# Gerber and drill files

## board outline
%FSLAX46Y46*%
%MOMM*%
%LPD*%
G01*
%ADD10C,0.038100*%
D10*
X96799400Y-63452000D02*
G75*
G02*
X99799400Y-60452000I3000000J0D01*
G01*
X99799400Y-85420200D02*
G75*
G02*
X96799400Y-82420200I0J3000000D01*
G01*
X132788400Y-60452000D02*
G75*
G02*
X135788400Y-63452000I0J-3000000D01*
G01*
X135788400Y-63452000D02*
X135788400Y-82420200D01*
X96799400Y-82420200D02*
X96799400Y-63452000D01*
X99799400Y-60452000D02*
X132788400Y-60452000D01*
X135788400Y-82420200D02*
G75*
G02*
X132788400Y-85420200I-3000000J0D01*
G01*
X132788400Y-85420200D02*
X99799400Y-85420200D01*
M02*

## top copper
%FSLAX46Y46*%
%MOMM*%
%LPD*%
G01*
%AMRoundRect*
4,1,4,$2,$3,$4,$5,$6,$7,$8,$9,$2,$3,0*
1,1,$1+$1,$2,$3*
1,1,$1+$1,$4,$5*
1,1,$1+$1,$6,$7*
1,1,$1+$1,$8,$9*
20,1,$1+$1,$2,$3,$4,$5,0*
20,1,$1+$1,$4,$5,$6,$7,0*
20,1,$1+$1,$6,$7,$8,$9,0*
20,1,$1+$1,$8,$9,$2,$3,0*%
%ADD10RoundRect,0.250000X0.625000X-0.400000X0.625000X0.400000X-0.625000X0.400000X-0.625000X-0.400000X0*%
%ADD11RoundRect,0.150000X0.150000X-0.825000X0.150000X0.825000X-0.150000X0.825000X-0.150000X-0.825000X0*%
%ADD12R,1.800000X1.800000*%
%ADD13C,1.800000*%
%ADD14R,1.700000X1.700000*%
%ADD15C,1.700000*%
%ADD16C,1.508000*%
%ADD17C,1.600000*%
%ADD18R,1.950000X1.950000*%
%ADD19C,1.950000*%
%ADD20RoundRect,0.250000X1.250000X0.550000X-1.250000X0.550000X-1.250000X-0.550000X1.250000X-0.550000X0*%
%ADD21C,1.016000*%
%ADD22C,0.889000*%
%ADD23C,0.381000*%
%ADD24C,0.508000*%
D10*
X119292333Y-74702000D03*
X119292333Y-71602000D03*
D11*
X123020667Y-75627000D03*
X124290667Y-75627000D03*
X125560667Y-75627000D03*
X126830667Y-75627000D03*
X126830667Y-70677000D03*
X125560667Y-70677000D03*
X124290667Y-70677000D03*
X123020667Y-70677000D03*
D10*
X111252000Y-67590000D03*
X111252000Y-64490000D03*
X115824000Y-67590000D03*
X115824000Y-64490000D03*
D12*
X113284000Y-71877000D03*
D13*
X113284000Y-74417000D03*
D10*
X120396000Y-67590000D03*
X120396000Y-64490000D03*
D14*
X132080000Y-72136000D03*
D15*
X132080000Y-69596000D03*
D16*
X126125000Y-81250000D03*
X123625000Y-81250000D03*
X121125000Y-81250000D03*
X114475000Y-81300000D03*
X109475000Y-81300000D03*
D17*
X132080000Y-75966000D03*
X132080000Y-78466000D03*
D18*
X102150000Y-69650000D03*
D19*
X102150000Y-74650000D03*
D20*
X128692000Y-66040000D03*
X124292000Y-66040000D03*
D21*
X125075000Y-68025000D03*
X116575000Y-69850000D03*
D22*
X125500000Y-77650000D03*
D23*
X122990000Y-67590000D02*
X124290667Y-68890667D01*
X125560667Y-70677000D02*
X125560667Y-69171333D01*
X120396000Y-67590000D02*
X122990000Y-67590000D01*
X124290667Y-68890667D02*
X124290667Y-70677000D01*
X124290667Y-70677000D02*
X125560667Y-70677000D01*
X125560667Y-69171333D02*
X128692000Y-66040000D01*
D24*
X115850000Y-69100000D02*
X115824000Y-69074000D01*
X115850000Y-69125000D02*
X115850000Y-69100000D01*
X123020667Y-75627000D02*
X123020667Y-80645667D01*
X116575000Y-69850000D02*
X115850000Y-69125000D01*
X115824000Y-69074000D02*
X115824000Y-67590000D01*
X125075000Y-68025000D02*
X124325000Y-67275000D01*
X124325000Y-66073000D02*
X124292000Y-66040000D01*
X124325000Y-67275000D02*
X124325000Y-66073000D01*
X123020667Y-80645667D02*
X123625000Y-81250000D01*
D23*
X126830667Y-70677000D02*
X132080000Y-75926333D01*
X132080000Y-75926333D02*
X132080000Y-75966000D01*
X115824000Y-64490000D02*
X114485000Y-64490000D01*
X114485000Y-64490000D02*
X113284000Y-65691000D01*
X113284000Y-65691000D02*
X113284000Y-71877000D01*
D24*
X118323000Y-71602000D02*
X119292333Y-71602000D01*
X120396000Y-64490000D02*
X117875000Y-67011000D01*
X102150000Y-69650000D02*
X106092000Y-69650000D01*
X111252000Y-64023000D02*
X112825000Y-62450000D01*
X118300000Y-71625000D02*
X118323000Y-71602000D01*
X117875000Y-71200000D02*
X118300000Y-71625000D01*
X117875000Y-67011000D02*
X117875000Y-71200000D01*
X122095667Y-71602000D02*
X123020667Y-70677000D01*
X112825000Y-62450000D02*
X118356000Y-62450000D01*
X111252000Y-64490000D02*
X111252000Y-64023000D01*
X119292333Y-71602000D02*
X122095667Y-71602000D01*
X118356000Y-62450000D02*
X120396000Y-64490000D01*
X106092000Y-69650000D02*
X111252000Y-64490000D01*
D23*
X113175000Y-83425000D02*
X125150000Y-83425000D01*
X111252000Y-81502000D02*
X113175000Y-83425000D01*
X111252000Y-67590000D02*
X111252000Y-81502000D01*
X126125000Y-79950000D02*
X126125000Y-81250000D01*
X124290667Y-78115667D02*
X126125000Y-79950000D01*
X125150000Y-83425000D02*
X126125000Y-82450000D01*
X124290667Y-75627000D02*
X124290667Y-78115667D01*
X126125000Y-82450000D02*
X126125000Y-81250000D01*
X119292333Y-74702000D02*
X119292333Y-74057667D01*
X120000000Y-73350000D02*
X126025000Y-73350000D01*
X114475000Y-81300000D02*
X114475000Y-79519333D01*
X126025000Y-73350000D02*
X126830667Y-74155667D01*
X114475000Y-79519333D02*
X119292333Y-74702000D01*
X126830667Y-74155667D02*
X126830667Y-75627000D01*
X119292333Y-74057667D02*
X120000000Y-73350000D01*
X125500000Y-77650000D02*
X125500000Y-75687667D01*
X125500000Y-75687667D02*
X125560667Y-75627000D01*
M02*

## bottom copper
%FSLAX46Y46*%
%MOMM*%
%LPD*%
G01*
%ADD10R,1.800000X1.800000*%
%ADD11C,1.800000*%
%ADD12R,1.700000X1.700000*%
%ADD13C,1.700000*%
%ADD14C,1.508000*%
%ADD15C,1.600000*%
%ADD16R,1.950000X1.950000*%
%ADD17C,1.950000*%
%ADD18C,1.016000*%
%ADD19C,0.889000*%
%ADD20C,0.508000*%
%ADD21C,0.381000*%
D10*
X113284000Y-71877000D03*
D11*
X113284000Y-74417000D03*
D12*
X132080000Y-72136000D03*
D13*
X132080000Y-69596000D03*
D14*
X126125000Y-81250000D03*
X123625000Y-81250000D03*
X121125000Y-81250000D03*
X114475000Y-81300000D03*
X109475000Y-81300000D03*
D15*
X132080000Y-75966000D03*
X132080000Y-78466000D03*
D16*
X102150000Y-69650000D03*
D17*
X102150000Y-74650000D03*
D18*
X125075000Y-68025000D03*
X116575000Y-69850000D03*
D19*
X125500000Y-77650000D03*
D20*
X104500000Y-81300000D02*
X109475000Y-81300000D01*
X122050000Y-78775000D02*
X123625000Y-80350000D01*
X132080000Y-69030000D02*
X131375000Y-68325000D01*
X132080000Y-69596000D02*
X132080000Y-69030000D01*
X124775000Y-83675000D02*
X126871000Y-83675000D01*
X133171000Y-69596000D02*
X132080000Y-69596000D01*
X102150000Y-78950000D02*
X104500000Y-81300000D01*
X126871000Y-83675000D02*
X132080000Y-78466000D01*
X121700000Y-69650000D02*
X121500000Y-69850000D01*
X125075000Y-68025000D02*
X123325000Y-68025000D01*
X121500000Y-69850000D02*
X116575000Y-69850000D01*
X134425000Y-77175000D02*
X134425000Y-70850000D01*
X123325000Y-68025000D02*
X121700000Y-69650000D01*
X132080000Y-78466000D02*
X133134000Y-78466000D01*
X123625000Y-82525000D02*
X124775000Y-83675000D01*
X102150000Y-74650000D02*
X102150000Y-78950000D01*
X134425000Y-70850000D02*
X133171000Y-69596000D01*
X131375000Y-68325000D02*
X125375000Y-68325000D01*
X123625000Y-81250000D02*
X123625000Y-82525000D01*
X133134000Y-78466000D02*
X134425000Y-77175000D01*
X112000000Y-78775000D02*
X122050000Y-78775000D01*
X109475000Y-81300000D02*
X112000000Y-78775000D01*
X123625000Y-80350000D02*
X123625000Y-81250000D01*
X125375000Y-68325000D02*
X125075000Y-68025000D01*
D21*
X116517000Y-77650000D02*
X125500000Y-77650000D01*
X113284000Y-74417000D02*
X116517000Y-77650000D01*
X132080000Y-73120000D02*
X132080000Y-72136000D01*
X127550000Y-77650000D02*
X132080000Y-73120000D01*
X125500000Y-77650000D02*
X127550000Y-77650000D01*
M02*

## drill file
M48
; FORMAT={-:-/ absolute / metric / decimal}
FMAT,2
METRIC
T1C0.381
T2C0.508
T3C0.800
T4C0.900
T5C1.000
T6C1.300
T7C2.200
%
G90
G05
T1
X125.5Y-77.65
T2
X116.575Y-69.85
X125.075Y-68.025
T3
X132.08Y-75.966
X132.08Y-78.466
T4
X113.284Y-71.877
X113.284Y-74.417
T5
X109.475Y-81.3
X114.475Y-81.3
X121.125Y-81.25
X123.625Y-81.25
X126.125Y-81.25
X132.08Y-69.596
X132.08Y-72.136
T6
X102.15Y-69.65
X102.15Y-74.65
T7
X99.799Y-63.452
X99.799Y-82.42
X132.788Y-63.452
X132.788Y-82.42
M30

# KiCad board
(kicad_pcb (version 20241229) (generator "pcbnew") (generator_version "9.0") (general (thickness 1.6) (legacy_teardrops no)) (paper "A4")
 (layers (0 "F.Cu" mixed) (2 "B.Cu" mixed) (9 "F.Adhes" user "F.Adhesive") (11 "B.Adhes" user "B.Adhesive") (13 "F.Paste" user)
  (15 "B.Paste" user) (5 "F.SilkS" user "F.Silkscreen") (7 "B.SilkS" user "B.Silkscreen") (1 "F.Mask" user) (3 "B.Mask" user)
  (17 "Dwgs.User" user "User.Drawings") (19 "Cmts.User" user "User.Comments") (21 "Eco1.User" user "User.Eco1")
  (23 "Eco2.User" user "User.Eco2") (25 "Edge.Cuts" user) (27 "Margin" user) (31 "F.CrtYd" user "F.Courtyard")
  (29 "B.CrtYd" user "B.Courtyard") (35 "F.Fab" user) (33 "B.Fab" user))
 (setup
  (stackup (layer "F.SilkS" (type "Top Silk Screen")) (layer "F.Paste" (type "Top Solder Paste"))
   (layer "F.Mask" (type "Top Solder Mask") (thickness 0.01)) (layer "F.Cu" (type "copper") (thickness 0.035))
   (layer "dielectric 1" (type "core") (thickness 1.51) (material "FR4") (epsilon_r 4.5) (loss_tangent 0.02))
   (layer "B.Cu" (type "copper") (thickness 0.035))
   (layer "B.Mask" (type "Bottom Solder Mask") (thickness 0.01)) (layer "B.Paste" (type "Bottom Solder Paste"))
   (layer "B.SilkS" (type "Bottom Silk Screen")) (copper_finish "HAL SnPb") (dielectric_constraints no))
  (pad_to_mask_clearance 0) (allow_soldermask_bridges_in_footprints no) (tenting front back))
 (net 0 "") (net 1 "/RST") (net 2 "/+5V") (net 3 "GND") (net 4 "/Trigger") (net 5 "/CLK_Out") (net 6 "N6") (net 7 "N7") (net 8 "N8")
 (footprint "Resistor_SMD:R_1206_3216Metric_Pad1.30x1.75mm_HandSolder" (layer "F.Cu") (at 119.292333 73.152 90)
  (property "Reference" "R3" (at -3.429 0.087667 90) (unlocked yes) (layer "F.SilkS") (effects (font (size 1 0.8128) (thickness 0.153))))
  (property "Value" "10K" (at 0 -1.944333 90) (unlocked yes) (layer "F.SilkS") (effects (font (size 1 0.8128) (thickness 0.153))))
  (pad "1" smd roundrect (at -1.55 0 90) (size 1.3 1.75) (layers "F.Cu" "F.Mask" "F.Paste") (roundrect_rratio 0.192308) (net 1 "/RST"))
  (pad "2" smd roundrect (at 1.55 0 90) (size 1.3 1.75) (layers "F.Cu" "F.Mask" "F.Paste") (roundrect_rratio 0.192308) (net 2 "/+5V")))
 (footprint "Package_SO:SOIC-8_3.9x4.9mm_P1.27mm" (layer "F.Cu") (at 124.925667 73.152 90)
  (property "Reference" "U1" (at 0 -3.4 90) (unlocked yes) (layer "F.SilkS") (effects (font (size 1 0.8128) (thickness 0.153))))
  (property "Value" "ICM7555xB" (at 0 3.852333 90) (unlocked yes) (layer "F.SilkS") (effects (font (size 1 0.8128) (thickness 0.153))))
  (pad "1" smd roundrect (at -2.475 -1.905 90) (size 1.95 0.6) (layers "F.Cu" "F.Mask" "F.Paste") (roundrect_rratio 0.25) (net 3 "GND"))
  (pad "2" smd roundrect (at -2.475 -0.635 90) (size 1.95 0.6) (layers "F.Cu" "F.Mask" "F.Paste") (roundrect_rratio 0.25) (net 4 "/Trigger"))
  (pad "3" smd roundrect (at -2.475 0.635 90) (size 1.95 0.6) (layers "F.Cu" "F.Mask" "F.Paste") (roundrect_rratio 0.25) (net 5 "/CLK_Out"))
  (pad "4" smd roundrect (at -2.475 1.905 90) (size 1.95 0.6) (layers "F.Cu" "F.Mask" "F.Paste") (roundrect_rratio 0.25) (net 1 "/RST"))
  (pad "5" smd roundrect (at 2.475 1.905 90) (size 1.95 0.6) (layers "F.Cu" "F.Mask" "F.Paste") (roundrect_rratio 0.25) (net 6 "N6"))
  (pad "6" smd roundrect (at 2.475 0.635 90) (size 1.95 0.6) (layers "F.Cu" "F.Mask" "F.Paste") (roundrect_rratio 0.25) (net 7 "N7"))
  (pad "7" smd roundrect (at 2.475 -0.635 90) (size 1.95 0.6) (layers "F.Cu" "F.Mask" "F.Paste") (roundrect_rratio 0.25) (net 7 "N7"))
  (pad "8" smd roundrect (at 2.475 -1.905 90) (size 1.95 0.6) (layers "F.Cu" "F.Mask" "F.Paste") (roundrect_rratio 0.25) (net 2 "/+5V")))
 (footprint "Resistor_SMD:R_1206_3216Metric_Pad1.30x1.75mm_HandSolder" (layer "F.Cu") (at 111.252 66.04 90)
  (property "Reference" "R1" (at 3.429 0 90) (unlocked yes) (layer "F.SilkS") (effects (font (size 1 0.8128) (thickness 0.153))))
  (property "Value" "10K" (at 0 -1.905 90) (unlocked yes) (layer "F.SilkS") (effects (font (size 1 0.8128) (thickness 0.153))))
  (pad "1" smd roundrect (at -1.55 0 90) (size 1.3 1.75) (layers "F.Cu" "F.Mask" "F.Paste") (roundrect_rratio 0.192308) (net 4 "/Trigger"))
  (pad "2" smd roundrect (at 1.55 0 90) (size 1.3 1.75) (layers "F.Cu" "F.Mask" "F.Paste") (roundrect_rratio 0.192308) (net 2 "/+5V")))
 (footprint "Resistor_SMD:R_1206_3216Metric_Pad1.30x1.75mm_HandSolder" (layer "F.Cu") (at 115.824 66.04 90)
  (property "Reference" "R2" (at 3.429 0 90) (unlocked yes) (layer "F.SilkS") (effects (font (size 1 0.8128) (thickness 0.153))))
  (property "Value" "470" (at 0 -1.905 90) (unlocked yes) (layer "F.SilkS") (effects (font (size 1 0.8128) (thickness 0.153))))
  (pad "1" smd roundrect (at -1.55 0 90) (size 1.3 1.75) (layers "F.Cu" "F.Mask" "F.Paste") (roundrect_rratio 0.192308) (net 3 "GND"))
  (pad "2" smd roundrect (at 1.55 0 90) (size 1.3 1.75) (layers "F.Cu" "F.Mask" "F.Paste") (roundrect_rratio 0.192308) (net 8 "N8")))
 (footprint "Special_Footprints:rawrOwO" (layer "F.Cu") (at 105.7 63.275)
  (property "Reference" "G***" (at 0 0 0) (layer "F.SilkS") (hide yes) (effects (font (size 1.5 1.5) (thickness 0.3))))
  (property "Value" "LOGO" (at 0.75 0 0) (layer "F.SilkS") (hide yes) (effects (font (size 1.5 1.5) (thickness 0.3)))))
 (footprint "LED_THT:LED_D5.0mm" (layer "F.Cu") (at 113.284 71.877 -90)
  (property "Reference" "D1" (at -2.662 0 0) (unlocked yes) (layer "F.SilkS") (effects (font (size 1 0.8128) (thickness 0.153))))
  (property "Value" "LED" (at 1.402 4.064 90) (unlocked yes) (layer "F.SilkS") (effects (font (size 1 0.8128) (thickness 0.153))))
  (pad "1" thru_hole rect (at 0 0 270) (size 1.8 1.8) (drill 0.9) (layers "*.Cu" "*.Mask") (remove_unused_layers no) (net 8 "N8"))
  (pad "2" thru_hole circle (at 2.54 0 270) (size 1.8 1.8) (drill 0.9) (layers "*.Cu" "*.Mask") (remove_unused_layers no) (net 5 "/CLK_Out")))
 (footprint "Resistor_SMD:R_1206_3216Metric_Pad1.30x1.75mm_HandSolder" (layer "F.Cu") (at 120.396 66.04 90)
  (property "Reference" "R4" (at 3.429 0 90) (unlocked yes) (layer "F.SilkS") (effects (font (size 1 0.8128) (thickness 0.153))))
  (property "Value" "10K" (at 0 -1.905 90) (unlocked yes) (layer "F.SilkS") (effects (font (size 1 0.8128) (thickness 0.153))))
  (pad "1" smd roundrect (at -1.55 0 90) (size 1.3 1.75) (layers "F.Cu" "F.Mask" "F.Paste") (roundrect_rratio 0.192308) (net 7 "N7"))
  (pad "2" smd roundrect (at 1.55 0 90) (size 1.3 1.75) (layers "F.Cu" "F.Mask" "F.Paste") (roundrect_rratio 0.192308) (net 2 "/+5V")))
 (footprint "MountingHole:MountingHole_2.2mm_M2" (layer "F.Cu") (at 99.7994 63.452)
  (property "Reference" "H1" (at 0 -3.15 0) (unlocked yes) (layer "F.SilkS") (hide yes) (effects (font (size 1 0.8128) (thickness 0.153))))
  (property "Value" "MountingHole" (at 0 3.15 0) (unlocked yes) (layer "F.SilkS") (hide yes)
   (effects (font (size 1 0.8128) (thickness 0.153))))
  (pad "" np_thru_hole circle (at 0 0) (size 2.2 2.2) (drill 2.2) (layers "*.Cu" "*.Mask")))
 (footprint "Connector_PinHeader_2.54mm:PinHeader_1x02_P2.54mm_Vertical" (layer "F.Cu") (at 132.08 72.136 180)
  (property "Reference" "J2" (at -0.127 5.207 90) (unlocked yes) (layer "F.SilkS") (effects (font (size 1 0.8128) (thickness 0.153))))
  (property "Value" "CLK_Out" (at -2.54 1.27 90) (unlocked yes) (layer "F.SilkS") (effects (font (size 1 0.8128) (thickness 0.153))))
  (pad "1" thru_hole rect (at 0 0 180) (size 1.7 1.7) (drill 1) (layers "*.Cu" "*.Mask") (remove_unused_layers no) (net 5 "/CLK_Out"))
  (pad "2" thru_hole circle (at 0 2.54 180) (size 1.7 1.7) (drill 1) (layers "*.Cu" "*.Mask") (remove_unused_layers no) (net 3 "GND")))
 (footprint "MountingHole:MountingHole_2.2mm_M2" (layer "F.Cu") (at 132.7884 82.4202)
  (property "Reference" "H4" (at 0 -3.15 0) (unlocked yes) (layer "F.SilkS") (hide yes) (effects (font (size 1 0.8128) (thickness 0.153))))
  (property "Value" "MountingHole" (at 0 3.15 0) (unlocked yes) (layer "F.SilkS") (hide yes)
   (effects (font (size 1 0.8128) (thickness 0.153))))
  (pad "" np_thru_hole circle (at 0 0) (size 2.2 2.2) (drill 2.2) (layers "*.Cu" "*.Mask")))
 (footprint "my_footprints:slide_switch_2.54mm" (layer "F.Cu") (at 123.625 81.25 180)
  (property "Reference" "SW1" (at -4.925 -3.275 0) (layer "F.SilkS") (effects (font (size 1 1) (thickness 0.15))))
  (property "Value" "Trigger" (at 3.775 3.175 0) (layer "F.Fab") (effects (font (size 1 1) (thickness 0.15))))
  (pad "1" thru_hole circle (at -2.5 0 180) (size 1.508 1.508) (drill 1) (layers "*.Cu" "*.Mask") (remove_unused_layers no)
   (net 4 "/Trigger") (solder_mask_margin 0.102))
  (pad "2" thru_hole circle (at 0 0 180) (size 1.508 1.508) (drill 1) (layers "*.Cu" "*.Mask") (remove_unused_layers no) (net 3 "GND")
   (solder_mask_margin 0.102))
  (pad "3" thru_hole circle (at 2.5 0 180) (size 1.508 1.508) (drill 1) (layers "*.Cu" "*.Mask") (remove_unused_layers no)
   (solder_mask_margin 0.102)))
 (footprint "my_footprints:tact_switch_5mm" (layer "F.Cu") (at 111.975 81.3 180)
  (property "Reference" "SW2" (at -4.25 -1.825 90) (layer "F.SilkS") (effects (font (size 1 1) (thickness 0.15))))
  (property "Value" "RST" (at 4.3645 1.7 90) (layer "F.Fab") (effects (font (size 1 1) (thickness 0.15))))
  (pad "1" thru_hole circle (at -2.5 0 180) (size 1.508 1.508) (drill 1) (layers "*.Cu" "*.Mask") (remove_unused_layers no) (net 1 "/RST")
   (solder_mask_margin 0.102))
  (pad "2" thru_hole circle (at 2.5 0 180) (size 1.508 1.508) (drill 1) (layers "*.Cu" "*.Mask") (remove_unused_layers no) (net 3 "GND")
   (solder_mask_margin 0.102)))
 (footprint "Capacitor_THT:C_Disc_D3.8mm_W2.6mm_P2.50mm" (layer "F.Cu") (at 132.08 75.966 -90)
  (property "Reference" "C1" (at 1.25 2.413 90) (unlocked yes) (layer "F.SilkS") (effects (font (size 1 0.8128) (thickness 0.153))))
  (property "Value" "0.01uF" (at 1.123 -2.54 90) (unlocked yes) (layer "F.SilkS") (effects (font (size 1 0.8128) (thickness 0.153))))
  (pad "1" thru_hole circle (at 0 0 270) (size 1.6 1.6) (drill 0.8) (layers "*.Cu" "*.Mask") (remove_unused_layers no) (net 6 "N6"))
  (pad "2" thru_hole circle (at 2.5 0 270) (size 1.6 1.6) (drill 0.8) (layers "*.Cu" "*.Mask") (remove_unused_layers no) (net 3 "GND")))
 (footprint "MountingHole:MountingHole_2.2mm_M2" (layer "F.Cu") (at 132.7884 63.452)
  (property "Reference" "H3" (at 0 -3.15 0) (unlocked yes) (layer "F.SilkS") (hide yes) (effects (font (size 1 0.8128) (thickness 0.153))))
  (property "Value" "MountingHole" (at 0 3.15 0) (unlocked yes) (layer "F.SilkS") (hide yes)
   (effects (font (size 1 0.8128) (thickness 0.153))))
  (pad "" np_thru_hole circle (at 0 0) (size 2.2 2.2) (drill 2.2) (layers "*.Cu" "*.Mask")))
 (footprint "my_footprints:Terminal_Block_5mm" (layer "F.Cu") (at 102.15 72.15 -90)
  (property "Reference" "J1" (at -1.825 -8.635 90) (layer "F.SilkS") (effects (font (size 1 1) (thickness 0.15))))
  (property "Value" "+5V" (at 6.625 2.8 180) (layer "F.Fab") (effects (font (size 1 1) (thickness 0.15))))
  (pad "1" thru_hole rect (at -2.5 0 270) (size 1.95 1.95) (drill 1.3) (layers "*.Cu" "*.Mask") (remove_unused_layers no) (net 2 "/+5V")
   (solder_mask_margin 0.102))
  (pad "2" thru_hole circle (at 2.5 0 270) (size 1.95 1.95) (drill 1.3) (layers "*.Cu" "*.Mask") (remove_unused_layers no) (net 3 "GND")
   (solder_mask_margin 0.102)))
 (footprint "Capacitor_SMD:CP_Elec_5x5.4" (layer "F.Cu") (at 126.492 66.04 180)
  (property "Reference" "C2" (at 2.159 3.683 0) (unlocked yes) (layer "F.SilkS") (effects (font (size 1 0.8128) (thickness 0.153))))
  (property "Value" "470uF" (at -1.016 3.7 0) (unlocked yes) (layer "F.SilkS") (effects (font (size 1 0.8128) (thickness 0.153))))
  (pad "1" smd roundrect (at -2.2 0 180) (size 3 1.6) (layers "F.Cu" "F.Mask" "F.Paste") (roundrect_rratio 0.15625) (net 7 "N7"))
  (pad "2" smd roundrect (at 2.2 0 180) (size 3 1.6) (layers "F.Cu" "F.Mask" "F.Paste") (roundrect_rratio 0.15625) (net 3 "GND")))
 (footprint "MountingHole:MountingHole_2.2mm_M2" (layer "F.Cu") (at 99.7994 82.4202)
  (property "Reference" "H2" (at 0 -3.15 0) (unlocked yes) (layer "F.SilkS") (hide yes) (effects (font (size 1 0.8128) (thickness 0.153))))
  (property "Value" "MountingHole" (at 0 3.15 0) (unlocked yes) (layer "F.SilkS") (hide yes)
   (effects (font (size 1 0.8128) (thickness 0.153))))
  (pad "" np_thru_hole circle (at 0 0) (size 2.2 2.2) (drill 2.2) (layers "*.Cu" "*.Mask")))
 (gr_arc (start 96.7994 63.452) (mid 97.67808 61.33068) (end 99.7994 60.452) (stroke (width 0.0381) (type default)) (layer "Edge.Cuts"))
 (gr_arc (start 99.7994 85.4202) (mid 97.67808 84.54152) (end 96.7994 82.4202) (stroke (width 0.0381) (type default)) (layer "Edge.Cuts"))
 (gr_arc (start 132.7884 60.452) (mid 134.90972 61.33068) (end 135.7884 63.452) (stroke (width 0.0381) (type default)) (layer "Edge.Cuts"))
 (gr_line (start 135.7884 63.452) (end 135.7884 82.4202) (stroke (width 0.0381) (type default)) (layer "Edge.Cuts"))
 (gr_line (start 96.7994 82.4202) (end 96.7994 63.452) (stroke (width 0.0381) (type default)) (layer "Edge.Cuts"))
 (gr_line (start 99.7994 60.452) (end 132.7884 60.452) (stroke (width 0.0381) (type default)) (layer "Edge.Cuts"))
 (gr_arc (start 135.7884 82.4202) (mid 134.90972 84.54152) (end 132.7884 85.4202) (stroke (width 0.0381) (type default)) (layer "Edge.Cuts"))
 (gr_line (start 132.7884 85.4202) (end 99.7994 85.4202) (stroke (width 0.0381) (type default)) (layer "Edge.Cuts"))
 (segment (start 122.99 67.59) (end 124.290667 68.890667) (width 0.381) (layer "F.Cu") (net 7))
 (segment (start 125.560667 70.677) (end 125.560667 69.171333) (width 0.381) (layer "F.Cu") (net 7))
 (segment (start 120.396 67.59) (end 122.99 67.59) (width 0.381) (layer "F.Cu") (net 7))
 (segment (start 124.290667 68.890667) (end 124.290667 70.677) (width 0.381) (layer "F.Cu") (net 7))
 (segment (start 124.290667 70.677) (end 125.560667 70.677) (width 0.381) (layer "F.Cu") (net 7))
 (segment (start 125.560667 69.171333) (end 128.692 66.04) (width 0.381) (layer "F.Cu") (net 7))
 (segment (start 115.85 69.1) (end 115.824 69.074) (width 0.508) (layer "F.Cu") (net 3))
 (segment (start 115.85 69.125) (end 115.85 69.1) (width 0.508) (layer "F.Cu") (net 3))
 (segment (start 123.020667 75.627) (end 123.020667 80.645667) (width 0.508) (layer "F.Cu") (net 3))
 (segment (start 116.575 69.85) (end 115.85 69.125) (width 0.508) (layer "F.Cu") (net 3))
 (segment (start 115.824 69.074) (end 115.824 67.59) (width 0.508) (layer "F.Cu") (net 3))
 (segment (start 125.075 68.025) (end 124.325 67.275) (width 0.508) (layer "F.Cu") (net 3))
 (segment (start 124.325 66.073) (end 124.292 66.04) (width 0.508) (layer "F.Cu") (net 3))
 (segment (start 124.325 67.275) (end 124.325 66.073) (width 0.508) (layer "F.Cu") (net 3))
 (segment (start 123.020667 80.645667) (end 123.625 81.25) (width 0.508) (layer "F.Cu") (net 3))
 (via (at 125.075 68.025) (size 1.016) (drill 0.508) (layers "F.Cu" "B.Cu") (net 3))
 (via (at 116.575 69.85) (size 1.016) (drill 0.508) (layers "F.Cu" "B.Cu") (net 3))
 (segment (start 104.5 81.3) (end 109.475 81.3) (width 0.508) (layer "B.Cu") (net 3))
 (segment (start 122.05 78.775) (end 123.625 80.35) (width 0.508) (layer "B.Cu") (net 3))
 (segment (start 132.08 69.03) (end 131.375 68.325) (width 0.508) (layer "B.Cu") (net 3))
 (segment (start 132.08 69.596) (end 132.08 69.03) (width 0.508) (layer "B.Cu") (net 3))
 (segment (start 124.775 83.675) (end 126.871 83.675) (width 0.508) (layer "B.Cu") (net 3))
 (segment (start 133.171 69.596) (end 132.08 69.596) (width 0.508) (layer "B.Cu") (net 3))
 (segment (start 102.15 78.95) (end 104.5 81.3) (width 0.508) (layer "B.Cu") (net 3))
 (segment (start 126.871 83.675) (end 132.08 78.466) (width 0.508) (layer "B.Cu") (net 3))
 (segment (start 121.7 69.65) (end 121.5 69.85) (width 0.508) (layer "B.Cu") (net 3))
 (segment (start 125.075 68.025) (end 123.325 68.025) (width 0.508) (layer "B.Cu") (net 3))
 (segment (start 121.5 69.85) (end 116.575 69.85) (width 0.508) (layer "B.Cu") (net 3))
 (segment (start 134.425 77.175) (end 134.425 70.85) (width 0.508) (layer "B.Cu") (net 3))
 (segment (start 123.325 68.025) (end 121.7 69.65) (width 0.508) (layer "B.Cu") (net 3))
 (segment (start 132.08 78.466) (end 133.134 78.466) (width 0.508) (layer "B.Cu") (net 3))
 (segment (start 123.625 82.525) (end 124.775 83.675) (width 0.508) (layer "B.Cu") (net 3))
 (segment (start 102.15 74.65) (end 102.15 78.95) (width 0.508) (layer "B.Cu") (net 3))
 (segment (start 134.425 70.85) (end 133.171 69.596) (width 0.508) (layer "B.Cu") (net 3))
 (segment (start 131.375 68.325) (end 125.375 68.325) (width 0.508) (layer "B.Cu") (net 3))
 (segment (start 123.625 81.25) (end 123.625 82.525) (width 0.508) (layer "B.Cu") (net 3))
 (segment (start 133.134 78.466) (end 134.425 77.175) (width 0.508) (layer "B.Cu") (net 3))
 (segment (start 112 78.775) (end 122.05 78.775) (width 0.508) (layer "B.Cu") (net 3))
 (segment (start 109.475 81.3) (end 112 78.775) (width 0.508) (layer "B.Cu") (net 3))
 (segment (start 123.625 80.35) (end 123.625 81.25) (width 0.508) (layer "B.Cu") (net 3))
 (segment (start 125.375 68.325) (end 125.075 68.025) (width 0.508) (layer "B.Cu") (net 3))
 (segment (start 126.830667 70.677) (end 132.08 75.926333) (width 0.381) (layer "F.Cu") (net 6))
 (segment (start 132.08 75.926333) (end 132.08 75.966) (width 0.381) (layer "F.Cu") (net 6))
 (segment (start 115.824 64.49) (end 114.485 64.49) (width 0.381) (layer "F.Cu") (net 8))
 (segment (start 114.485 64.49) (end 113.284 65.691) (width 0.381) (layer "F.Cu") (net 8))
 (segment (start 113.284 65.691) (end 113.284 71.877) (width 0.381) (layer "F.Cu") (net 8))
 (segment (start 118.323 71.602) (end 119.292333 71.602) (width 0.508) (layer "F.Cu") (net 2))
 (segment (start 120.396 64.49) (end 117.875 67.011) (width 0.508) (layer "F.Cu") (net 2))
 (segment (start 102.15 69.65) (end 106.092 69.65) (width 0.508) (layer "F.Cu") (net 2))
 (segment (start 111.252 64.023) (end 112.825 62.45) (width 0.508) (layer "F.Cu") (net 2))
 (segment (start 118.3 71.625) (end 118.323 71.602) (width 0.508) (layer "F.Cu") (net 2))
 (segment (start 117.875 71.2) (end 118.3 71.625) (width 0.508) (layer "F.Cu") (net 2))
 (segment (start 117.875 67.011) (end 117.875 71.2) (width 0.508) (layer "F.Cu") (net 2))
 (segment (start 122.095667 71.602) (end 123.020667 70.677) (width 0.508) (layer "F.Cu") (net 2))
 (segment (start 112.825 62.45) (end 118.356 62.45) (width 0.508) (layer "F.Cu") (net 2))
 (segment (start 111.252 64.49) (end 111.252 64.023) (width 0.508) (layer "F.Cu") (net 2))
 (segment (start 119.292333 71.602) (end 122.095667 71.602) (width 0.508) (layer "F.Cu") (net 2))
 (segment (start 118.356 62.45) (end 120.396 64.49) (width 0.508) (layer "F.Cu") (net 2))
 (segment (start 106.092 69.65) (end 111.252 64.49) (width 0.508) (layer "F.Cu") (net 2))
 (segment (start 113.175 83.425) (end 125.15 83.425) (width 0.381) (layer "F.Cu") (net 4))
 (segment (start 111.252 81.502) (end 113.175 83.425) (width 0.381) (layer "F.Cu") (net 4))
 (segment (start 111.252 67.59) (end 111.252 81.502) (width 0.381) (layer "F.Cu") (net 4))
 (segment (start 126.125 79.95) (end 126.125 81.25) (width 0.381) (layer "F.Cu") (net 4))
 (segment (start 124.290667 78.115667) (end 126.125 79.95) (width 0.381) (layer "F.Cu") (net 4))
 (segment (start 125.15 83.425) (end 126.125 82.45) (width 0.381) (layer "F.Cu") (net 4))
 (segment (start 124.290667 75.627) (end 124.290667 78.115667) (width 0.381) (layer "F.Cu") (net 4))
 (segment (start 126.125 82.45) (end 126.125 81.25) (width 0.381) (layer "F.Cu") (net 4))
 (segment (start 119.292333 74.702) (end 119.292333 74.057667) (width 0.381) (layer "F.Cu") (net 1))
 (segment (start 120 73.35) (end 126.025 73.35) (width 0.381) (layer "F.Cu") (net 1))
 (segment (start 114.475 81.3) (end 114.475 79.519333) (width 0.381) (layer "F.Cu") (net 1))
 (segment (start 126.025 73.35) (end 126.830667 74.155667) (width 0.381) (layer "F.Cu") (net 1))
 (segment (start 114.475 79.519333) (end 119.292333 74.702) (width 0.381) (layer "F.Cu") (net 1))
 (segment (start 126.830667 74.155667) (end 126.830667 75.627) (width 0.381) (layer "F.Cu") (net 1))
 (segment (start 119.292333 74.057667) (end 120 73.35) (width 0.381) (layer "F.Cu") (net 1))
 (segment (start 125.5 77.65) (end 125.5 75.687667) (width 0.381) (layer "F.Cu") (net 5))
 (segment (start 125.5 75.687667) (end 125.560667 75.627) (width 0.381) (layer "F.Cu") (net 5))
 (via (at 125.5 77.65) (size 0.889) (drill 0.381) (layers "F.Cu" "B.Cu") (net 5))
 (segment (start 116.517 77.65) (end 125.5 77.65) (width 0.381) (layer "B.Cu") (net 5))
 (segment (start 113.284 74.417) (end 116.517 77.65) (width 0.381) (layer "B.Cu") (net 5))
 (segment (start 132.08 73.12) (end 132.08 72.136) (width 0.381) (layer "B.Cu") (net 5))
 (segment (start 127.55 77.65) (end 132.08 73.12) (width 0.381) (layer "B.Cu") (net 5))
 (segment (start 125.5 77.65) (end 127.55 77.65) (width 0.381) (layer "B.Cu") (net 5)))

